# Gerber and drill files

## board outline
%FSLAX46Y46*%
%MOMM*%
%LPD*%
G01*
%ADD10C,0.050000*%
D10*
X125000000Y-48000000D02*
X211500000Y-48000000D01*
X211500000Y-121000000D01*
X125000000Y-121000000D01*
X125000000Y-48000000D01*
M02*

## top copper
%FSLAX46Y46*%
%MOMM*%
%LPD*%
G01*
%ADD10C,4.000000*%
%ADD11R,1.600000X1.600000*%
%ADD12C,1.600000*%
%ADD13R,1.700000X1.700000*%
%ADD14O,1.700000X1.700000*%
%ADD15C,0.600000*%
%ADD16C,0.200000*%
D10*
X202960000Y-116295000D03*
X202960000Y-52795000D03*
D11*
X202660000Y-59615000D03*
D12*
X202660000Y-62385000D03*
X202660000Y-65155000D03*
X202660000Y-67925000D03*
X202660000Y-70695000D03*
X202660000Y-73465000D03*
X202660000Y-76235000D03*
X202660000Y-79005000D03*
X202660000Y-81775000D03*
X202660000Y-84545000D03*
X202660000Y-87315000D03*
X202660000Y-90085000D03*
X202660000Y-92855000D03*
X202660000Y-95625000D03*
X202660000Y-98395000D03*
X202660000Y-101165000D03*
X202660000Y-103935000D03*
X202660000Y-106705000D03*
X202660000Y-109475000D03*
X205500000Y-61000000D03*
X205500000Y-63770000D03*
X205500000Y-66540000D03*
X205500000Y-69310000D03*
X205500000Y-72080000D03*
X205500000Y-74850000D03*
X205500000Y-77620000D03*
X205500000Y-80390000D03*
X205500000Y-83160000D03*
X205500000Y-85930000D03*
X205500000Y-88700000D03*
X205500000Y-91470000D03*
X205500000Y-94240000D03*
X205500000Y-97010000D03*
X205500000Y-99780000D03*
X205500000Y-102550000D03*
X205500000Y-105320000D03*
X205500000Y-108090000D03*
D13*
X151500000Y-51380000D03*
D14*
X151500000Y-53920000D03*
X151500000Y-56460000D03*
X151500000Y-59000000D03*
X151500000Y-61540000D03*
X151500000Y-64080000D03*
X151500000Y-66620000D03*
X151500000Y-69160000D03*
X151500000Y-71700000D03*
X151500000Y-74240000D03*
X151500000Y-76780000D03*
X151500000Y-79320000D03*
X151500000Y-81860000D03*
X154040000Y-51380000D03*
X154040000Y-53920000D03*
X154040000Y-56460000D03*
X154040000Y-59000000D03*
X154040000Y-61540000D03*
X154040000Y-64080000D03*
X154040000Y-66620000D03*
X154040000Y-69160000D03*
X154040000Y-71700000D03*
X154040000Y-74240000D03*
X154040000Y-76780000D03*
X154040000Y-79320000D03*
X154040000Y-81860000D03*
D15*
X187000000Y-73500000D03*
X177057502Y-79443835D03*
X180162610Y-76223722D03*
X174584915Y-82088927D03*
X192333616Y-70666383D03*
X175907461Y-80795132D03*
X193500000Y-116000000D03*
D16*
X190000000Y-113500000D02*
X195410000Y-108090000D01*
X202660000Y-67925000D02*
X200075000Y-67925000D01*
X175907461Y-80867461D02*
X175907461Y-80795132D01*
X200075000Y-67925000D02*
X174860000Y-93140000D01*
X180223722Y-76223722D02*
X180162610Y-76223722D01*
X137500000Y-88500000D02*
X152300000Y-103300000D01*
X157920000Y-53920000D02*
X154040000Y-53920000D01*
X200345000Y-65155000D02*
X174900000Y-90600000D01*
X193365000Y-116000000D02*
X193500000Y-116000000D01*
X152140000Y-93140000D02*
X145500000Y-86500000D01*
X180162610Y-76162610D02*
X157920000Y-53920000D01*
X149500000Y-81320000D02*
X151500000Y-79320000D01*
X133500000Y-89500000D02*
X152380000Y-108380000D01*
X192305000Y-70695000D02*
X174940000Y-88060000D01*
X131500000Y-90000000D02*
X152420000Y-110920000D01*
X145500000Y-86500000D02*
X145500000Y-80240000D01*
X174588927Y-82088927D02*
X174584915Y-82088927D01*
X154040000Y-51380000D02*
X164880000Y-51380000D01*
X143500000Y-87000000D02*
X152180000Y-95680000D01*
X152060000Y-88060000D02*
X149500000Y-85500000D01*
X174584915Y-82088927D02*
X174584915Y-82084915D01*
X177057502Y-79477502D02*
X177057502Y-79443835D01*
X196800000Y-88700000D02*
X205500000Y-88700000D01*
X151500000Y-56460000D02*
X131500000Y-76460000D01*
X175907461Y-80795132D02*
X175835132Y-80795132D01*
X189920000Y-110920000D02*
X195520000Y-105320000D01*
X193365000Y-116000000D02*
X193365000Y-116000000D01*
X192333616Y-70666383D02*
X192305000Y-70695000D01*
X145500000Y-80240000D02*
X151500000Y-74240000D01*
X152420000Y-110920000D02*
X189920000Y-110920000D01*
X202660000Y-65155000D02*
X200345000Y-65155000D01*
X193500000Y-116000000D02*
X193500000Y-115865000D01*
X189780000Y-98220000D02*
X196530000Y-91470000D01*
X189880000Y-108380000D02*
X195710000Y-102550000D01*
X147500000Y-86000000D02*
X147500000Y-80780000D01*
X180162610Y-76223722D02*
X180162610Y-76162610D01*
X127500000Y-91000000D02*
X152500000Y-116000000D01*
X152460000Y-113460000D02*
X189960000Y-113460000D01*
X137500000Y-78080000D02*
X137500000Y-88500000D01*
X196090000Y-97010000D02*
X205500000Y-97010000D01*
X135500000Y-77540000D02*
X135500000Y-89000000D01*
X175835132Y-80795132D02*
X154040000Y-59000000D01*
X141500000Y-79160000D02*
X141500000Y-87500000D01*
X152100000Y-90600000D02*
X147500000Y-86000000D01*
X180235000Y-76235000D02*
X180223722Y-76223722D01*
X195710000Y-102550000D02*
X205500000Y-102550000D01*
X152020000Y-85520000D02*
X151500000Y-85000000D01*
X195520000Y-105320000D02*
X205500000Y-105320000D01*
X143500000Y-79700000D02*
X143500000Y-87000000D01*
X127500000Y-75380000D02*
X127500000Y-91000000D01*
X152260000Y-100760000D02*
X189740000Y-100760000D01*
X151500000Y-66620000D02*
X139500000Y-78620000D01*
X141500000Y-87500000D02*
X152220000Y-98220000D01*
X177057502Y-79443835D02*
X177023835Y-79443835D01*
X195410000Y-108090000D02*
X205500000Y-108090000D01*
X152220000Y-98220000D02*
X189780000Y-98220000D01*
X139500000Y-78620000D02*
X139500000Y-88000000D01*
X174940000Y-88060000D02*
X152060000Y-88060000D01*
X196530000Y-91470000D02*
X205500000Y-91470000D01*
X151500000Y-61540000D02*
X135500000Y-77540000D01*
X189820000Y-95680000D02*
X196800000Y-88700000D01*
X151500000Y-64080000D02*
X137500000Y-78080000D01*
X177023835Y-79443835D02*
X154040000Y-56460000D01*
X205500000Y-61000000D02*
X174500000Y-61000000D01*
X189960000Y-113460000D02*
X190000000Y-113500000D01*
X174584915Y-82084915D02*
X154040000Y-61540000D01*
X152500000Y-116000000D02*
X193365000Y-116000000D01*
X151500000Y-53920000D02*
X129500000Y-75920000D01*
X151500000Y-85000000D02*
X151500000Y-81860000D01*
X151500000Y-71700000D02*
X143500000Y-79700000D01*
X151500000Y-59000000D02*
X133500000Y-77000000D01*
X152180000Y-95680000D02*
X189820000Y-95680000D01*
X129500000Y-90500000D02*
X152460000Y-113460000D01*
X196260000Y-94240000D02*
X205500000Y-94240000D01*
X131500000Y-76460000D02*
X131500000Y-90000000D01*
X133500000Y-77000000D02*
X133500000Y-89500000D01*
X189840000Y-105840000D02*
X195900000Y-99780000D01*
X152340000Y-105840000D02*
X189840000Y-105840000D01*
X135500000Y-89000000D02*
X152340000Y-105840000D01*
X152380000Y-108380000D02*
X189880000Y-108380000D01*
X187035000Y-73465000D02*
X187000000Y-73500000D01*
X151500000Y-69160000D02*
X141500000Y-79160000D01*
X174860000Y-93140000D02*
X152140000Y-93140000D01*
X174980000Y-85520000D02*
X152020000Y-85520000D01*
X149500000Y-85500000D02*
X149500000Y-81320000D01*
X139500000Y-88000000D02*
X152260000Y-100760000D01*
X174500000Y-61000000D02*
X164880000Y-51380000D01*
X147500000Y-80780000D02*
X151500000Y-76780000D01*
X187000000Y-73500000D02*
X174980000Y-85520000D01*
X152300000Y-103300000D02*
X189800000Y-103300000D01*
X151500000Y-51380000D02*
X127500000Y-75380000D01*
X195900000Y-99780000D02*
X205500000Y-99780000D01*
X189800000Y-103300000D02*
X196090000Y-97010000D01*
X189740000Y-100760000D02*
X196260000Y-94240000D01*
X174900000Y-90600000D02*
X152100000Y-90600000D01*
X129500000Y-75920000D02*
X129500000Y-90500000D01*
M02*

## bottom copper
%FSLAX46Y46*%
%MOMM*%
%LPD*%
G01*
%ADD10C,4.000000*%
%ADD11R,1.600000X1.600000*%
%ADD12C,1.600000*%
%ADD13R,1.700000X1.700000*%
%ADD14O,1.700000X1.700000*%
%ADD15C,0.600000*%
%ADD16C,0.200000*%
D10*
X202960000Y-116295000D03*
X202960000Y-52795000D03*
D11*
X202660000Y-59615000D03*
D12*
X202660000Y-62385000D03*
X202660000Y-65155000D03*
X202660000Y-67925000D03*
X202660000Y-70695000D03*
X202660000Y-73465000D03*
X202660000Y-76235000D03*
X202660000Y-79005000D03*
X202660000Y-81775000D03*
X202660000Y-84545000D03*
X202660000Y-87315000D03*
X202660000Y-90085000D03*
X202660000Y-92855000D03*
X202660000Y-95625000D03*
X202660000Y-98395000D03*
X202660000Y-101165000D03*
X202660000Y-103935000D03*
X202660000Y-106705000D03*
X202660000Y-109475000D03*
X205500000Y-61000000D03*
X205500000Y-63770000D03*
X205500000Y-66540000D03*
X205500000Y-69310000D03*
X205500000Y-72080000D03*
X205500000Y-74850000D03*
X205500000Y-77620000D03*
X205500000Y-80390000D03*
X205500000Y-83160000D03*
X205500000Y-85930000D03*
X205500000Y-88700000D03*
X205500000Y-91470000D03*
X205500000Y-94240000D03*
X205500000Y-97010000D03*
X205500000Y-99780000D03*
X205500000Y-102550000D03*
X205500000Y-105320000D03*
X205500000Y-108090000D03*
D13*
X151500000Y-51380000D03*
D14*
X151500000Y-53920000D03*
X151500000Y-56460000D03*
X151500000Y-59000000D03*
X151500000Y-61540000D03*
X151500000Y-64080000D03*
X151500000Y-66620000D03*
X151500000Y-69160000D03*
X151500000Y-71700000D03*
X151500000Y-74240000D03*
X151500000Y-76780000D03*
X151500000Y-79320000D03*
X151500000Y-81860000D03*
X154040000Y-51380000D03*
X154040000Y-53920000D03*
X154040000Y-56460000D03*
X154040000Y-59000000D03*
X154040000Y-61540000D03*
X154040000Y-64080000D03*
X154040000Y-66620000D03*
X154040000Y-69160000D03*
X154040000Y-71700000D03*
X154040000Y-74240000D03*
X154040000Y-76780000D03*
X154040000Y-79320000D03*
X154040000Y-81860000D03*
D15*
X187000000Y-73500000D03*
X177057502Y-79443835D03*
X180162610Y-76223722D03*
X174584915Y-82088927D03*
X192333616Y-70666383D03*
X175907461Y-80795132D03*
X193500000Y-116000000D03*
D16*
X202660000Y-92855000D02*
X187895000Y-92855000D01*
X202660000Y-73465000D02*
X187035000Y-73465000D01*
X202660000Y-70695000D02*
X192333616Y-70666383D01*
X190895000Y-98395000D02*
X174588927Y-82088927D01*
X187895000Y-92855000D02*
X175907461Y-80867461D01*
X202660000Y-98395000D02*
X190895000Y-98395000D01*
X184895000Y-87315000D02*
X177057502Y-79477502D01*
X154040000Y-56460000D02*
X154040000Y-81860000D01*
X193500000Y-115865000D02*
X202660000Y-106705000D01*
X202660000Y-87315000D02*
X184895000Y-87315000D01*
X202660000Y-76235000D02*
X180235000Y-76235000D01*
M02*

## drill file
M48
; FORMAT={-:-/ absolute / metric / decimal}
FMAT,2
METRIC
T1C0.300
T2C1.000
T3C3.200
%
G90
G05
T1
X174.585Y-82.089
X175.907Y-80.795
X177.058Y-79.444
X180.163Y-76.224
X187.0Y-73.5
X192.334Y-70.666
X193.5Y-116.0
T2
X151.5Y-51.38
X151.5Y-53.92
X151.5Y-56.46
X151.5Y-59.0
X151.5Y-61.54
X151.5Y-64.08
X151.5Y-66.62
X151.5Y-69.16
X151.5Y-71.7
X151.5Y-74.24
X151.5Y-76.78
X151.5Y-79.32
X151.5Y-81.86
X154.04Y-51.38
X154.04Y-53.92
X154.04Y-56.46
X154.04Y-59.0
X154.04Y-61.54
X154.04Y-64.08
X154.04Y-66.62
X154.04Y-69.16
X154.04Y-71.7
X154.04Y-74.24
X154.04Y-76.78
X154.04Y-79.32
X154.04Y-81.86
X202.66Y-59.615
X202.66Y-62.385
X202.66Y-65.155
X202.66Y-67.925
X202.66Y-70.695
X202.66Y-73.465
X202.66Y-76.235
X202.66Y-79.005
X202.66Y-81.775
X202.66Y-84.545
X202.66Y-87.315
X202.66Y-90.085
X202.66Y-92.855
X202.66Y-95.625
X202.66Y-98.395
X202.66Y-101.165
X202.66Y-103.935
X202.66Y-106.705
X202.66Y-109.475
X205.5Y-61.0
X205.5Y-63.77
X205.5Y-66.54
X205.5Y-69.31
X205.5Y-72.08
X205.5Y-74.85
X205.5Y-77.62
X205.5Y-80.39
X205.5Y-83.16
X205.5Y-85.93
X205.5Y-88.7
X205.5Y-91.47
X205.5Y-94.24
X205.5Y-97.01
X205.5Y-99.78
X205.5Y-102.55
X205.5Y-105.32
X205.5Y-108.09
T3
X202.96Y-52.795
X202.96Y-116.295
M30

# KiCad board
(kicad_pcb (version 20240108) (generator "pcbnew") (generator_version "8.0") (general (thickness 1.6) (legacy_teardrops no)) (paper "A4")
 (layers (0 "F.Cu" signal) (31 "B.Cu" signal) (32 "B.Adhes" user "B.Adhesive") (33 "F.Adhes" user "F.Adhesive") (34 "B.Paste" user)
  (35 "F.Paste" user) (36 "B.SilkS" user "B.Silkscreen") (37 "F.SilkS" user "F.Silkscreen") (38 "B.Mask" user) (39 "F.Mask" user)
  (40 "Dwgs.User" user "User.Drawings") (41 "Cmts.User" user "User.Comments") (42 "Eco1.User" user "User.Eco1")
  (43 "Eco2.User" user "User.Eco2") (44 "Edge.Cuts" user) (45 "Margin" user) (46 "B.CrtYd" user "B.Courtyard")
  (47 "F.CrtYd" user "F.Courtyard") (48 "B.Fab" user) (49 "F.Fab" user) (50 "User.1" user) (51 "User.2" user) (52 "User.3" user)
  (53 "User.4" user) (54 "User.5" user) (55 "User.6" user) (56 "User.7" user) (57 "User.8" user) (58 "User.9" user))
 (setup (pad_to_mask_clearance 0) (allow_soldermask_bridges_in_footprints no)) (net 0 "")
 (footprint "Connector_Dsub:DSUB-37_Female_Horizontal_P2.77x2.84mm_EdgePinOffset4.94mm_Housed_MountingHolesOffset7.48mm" (layer "F.Cu")
  (at 202.66 59.615 90)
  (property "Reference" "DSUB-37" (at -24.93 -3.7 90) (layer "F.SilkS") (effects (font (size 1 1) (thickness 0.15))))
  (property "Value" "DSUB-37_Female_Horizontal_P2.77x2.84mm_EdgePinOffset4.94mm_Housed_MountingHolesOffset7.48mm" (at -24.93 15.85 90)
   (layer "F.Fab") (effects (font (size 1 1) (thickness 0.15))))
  (pad "0" thru_hole circle (at -56.68 0.3 90) (size 4 4) (drill 3.2) (layers "*.Cu" "*.Mask") (remove_unused_layers no))
  (pad "0" thru_hole circle (at 6.82 0.3 90) (size 4 4) (drill 3.2) (layers "*.Cu" "*.Mask") (remove_unused_layers no))
  (pad "1" thru_hole rect (at 0 0 90) (size 1.6 1.6) (drill 1) (layers "*.Cu" "*.Mask") (remove_unused_layers no))
  (pad "2" thru_hole circle (at -2.77 0 90) (size 1.6 1.6) (drill 1) (layers "*.Cu" "*.Mask") (remove_unused_layers no))
  (pad "3" thru_hole circle (at -5.54 0 90) (size 1.6 1.6) (drill 1) (layers "*.Cu" "*.Mask") (remove_unused_layers no))
  (pad "4" thru_hole circle (at -8.31 0 90) (size 1.6 1.6) (drill 1) (layers "*.Cu" "*.Mask") (remove_unused_layers no))
  (pad "5" thru_hole circle (at -11.08 0 90) (size 1.6 1.6) (drill 1) (layers "*.Cu" "*.Mask") (remove_unused_layers no))
  (pad "6" thru_hole circle (at -13.85 0 90) (size 1.6 1.6) (drill 1) (layers "*.Cu" "*.Mask") (remove_unused_layers no))
  (pad "7" thru_hole circle (at -16.62 0 90) (size 1.6 1.6) (drill 1) (layers "*.Cu" "*.Mask") (remove_unused_layers no))
  (pad "8" thru_hole circle (at -19.39 0 90) (size 1.6 1.6) (drill 1) (layers "*.Cu" "*.Mask") (remove_unused_layers no))
  (pad "9" thru_hole circle (at -22.16 0 90) (size 1.6 1.6) (drill 1) (layers "*.Cu" "*.Mask") (remove_unused_layers no))
  (pad "10" thru_hole circle (at -24.93 0 90) (size 1.6 1.6) (drill 1) (layers "*.Cu" "*.Mask") (remove_unused_layers no))
  (pad "11" thru_hole circle (at -27.7 0 90) (size 1.6 1.6) (drill 1) (layers "*.Cu" "*.Mask") (remove_unused_layers no))
  (pad "12" thru_hole circle (at -30.47 0 90) (size 1.6 1.6) (drill 1) (layers "*.Cu" "*.Mask") (remove_unused_layers no))
  (pad "13" thru_hole circle (at -33.24 0 90) (size 1.6 1.6) (drill 1) (layers "*.Cu" "*.Mask") (remove_unused_layers no))
  (pad "14" thru_hole circle (at -36.01 0 90) (size 1.6 1.6) (drill 1) (layers "*.Cu" "*.Mask") (remove_unused_layers no))
  (pad "15" thru_hole circle (at -38.78 0 90) (size 1.6 1.6) (drill 1) (layers "*.Cu" "*.Mask") (remove_unused_layers no))
  (pad "16" thru_hole circle (at -41.55 0 90) (size 1.6 1.6) (drill 1) (layers "*.Cu" "*.Mask") (remove_unused_layers no))
  (pad "17" thru_hole circle (at -44.32 0 90) (size 1.6 1.6) (drill 1) (layers "*.Cu" "*.Mask") (remove_unused_layers no))
  (pad "18" thru_hole circle (at -47.09 0 90) (size 1.6 1.6) (drill 1) (layers "*.Cu" "*.Mask") (remove_unused_layers no))
  (pad "19" thru_hole circle (at -49.86 0 90) (size 1.6 1.6) (drill 1) (layers "*.Cu" "*.Mask") (remove_unused_layers no))
  (pad "20" thru_hole circle (at -1.385 2.84 90) (size 1.6 1.6) (drill 1) (layers "*.Cu" "*.Mask") (remove_unused_layers no))
  (pad "21" thru_hole circle (at -4.155 2.84 90) (size 1.6 1.6) (drill 1) (layers "*.Cu" "*.Mask") (remove_unused_layers no))
  (pad "22" thru_hole circle (at -6.925 2.84 90) (size 1.6 1.6) (drill 1) (layers "*.Cu" "*.Mask") (remove_unused_layers no))
  (pad "23" thru_hole circle (at -9.695 2.84 90) (size 1.6 1.6) (drill 1) (layers "*.Cu" "*.Mask") (remove_unused_layers no))
  (pad "24" thru_hole circle (at -12.465 2.84 90) (size 1.6 1.6) (drill 1) (layers "*.Cu" "*.Mask") (remove_unused_layers no))
  (pad "25" thru_hole circle (at -15.235 2.84 90) (size 1.6 1.6) (drill 1) (layers "*.Cu" "*.Mask") (remove_unused_layers no))
  (pad "26" thru_hole circle (at -18.005 2.84 90) (size 1.6 1.6) (drill 1) (layers "*.Cu" "*.Mask") (remove_unused_layers no))
  (pad "27" thru_hole circle (at -20.775 2.84 90) (size 1.6 1.6) (drill 1) (layers "*.Cu" "*.Mask") (remove_unused_layers no))
  (pad "28" thru_hole circle (at -23.545 2.84 90) (size 1.6 1.6) (drill 1) (layers "*.Cu" "*.Mask") (remove_unused_layers no))
  (pad "29" thru_hole circle (at -26.315 2.84 90) (size 1.6 1.6) (drill 1) (layers "*.Cu" "*.Mask") (remove_unused_layers no))
  (pad "30" thru_hole circle (at -29.085 2.84 90) (size 1.6 1.6) (drill 1) (layers "*.Cu" "*.Mask") (remove_unused_layers no))
  (pad "31" thru_hole circle (at -31.855 2.84 90) (size 1.6 1.6) (drill 1) (layers "*.Cu" "*.Mask") (remove_unused_layers no))
  (pad "32" thru_hole circle (at -34.625 2.84 90) (size 1.6 1.6) (drill 1) (layers "*.Cu" "*.Mask") (remove_unused_layers no))
  (pad "33" thru_hole circle (at -37.395 2.84 90) (size 1.6 1.6) (drill 1) (layers "*.Cu" "*.Mask") (remove_unused_layers no))
  (pad "34" thru_hole circle (at -40.165 2.84 90) (size 1.6 1.6) (drill 1) (layers "*.Cu" "*.Mask") (remove_unused_layers no))
  (pad "35" thru_hole circle (at -42.935 2.84 90) (size 1.6 1.6) (drill 1) (layers "*.Cu" "*.Mask") (remove_unused_layers no))
  (pad "36" thru_hole circle (at -45.705 2.84 90) (size 1.6 1.6) (drill 1) (layers "*.Cu" "*.Mask") (remove_unused_layers no))
  (pad "37" thru_hole circle (at -48.475 2.84 90) (size 1.6 1.6) (drill 1) (layers "*.Cu" "*.Mask") (remove_unused_layers no)))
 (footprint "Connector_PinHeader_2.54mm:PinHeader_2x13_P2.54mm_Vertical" (layer "F.Cu") (at 151.5 51.38)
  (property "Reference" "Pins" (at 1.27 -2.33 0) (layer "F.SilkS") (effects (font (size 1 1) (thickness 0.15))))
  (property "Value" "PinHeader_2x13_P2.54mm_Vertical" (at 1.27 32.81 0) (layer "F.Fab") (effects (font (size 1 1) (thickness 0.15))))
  (pad "1" thru_hole rect (at 0 0) (size 1.7 1.7) (drill 1) (layers "*.Cu" "*.Mask") (remove_unused_layers no))
  (pad "2" thru_hole oval (at 0 2.54) (size 1.7 1.7) (drill 1) (layers "*.Cu" "*.Mask") (remove_unused_layers no))
  (pad "3" thru_hole oval (at 0 5.08) (size 1.7 1.7) (drill 1) (layers "*.Cu" "*.Mask") (remove_unused_layers no))
  (pad "4" thru_hole oval (at 0 7.62) (size 1.7 1.7) (drill 1) (layers "*.Cu" "*.Mask") (remove_unused_layers no))
  (pad "5" thru_hole oval (at 0 10.16) (size 1.7 1.7) (drill 1) (layers "*.Cu" "*.Mask") (remove_unused_layers no))
  (pad "6" thru_hole oval (at 0 12.7) (size 1.7 1.7) (drill 1) (layers "*.Cu" "*.Mask") (remove_unused_layers no))
  (pad "7" thru_hole oval (at 0 15.24) (size 1.7 1.7) (drill 1) (layers "*.Cu" "*.Mask") (remove_unused_layers no))
  (pad "8" thru_hole oval (at 0 17.78) (size 1.7 1.7) (drill 1) (layers "*.Cu" "*.Mask") (remove_unused_layers no))
  (pad "9" thru_hole oval (at 0 20.32) (size 1.7 1.7) (drill 1) (layers "*.Cu" "*.Mask") (remove_unused_layers no))
  (pad "10" thru_hole oval (at 0 22.86) (size 1.7 1.7) (drill 1) (layers "*.Cu" "*.Mask") (remove_unused_layers no))
  (pad "11" thru_hole oval (at 0 25.4) (size 1.7 1.7) (drill 1) (layers "*.Cu" "*.Mask") (remove_unused_layers no))
  (pad "12" thru_hole oval (at 0 27.94) (size 1.7 1.7) (drill 1) (layers "*.Cu" "*.Mask") (remove_unused_layers no))
  (pad "13" thru_hole oval (at 0 30.48) (size 1.7 1.7) (drill 1) (layers "*.Cu" "*.Mask") (remove_unused_layers no))
  (pad "14" thru_hole oval (at 2.54 0) (size 1.7 1.7) (drill 1) (layers "*.Cu" "*.Mask") (remove_unused_layers no))
  (pad "15" thru_hole oval (at 2.54 2.54) (size 1.7 1.7) (drill 1) (layers "*.Cu" "*.Mask") (remove_unused_layers no))
  (pad "16" thru_hole oval (at 2.54 5.08) (size 1.7 1.7) (drill 1) (layers "*.Cu" "*.Mask") (remove_unused_layers no))
  (pad "17" thru_hole oval (at 2.54 7.62) (size 1.7 1.7) (drill 1) (layers "*.Cu" "*.Mask") (remove_unused_layers no))
  (pad "18" thru_hole oval (at 2.54 10.16) (size 1.7 1.7) (drill 1) (layers "*.Cu" "*.Mask") (remove_unused_layers no))
  (pad "19" thru_hole oval (at 2.54 12.7) (size 1.7 1.7) (drill 1) (layers "*.Cu" "*.Mask") (remove_unused_layers no))
  (pad "20" thru_hole oval (at 2.54 15.24) (size 1.7 1.7) (drill 1) (layers "*.Cu" "*.Mask") (remove_unused_layers no))
  (pad "21" thru_hole oval (at 2.54 17.78) (size 1.7 1.7) (drill 1) (layers "*.Cu" "*.Mask") (remove_unused_layers no))
  (pad "22" thru_hole oval (at 2.54 20.32) (size 1.7 1.7) (drill 1) (layers "*.Cu" "*.Mask") (remove_unused_layers no))
  (pad "23" thru_hole oval (at 2.54 22.86) (size 1.7 1.7) (drill 1) (layers "*.Cu" "*.Mask") (remove_unused_layers no))
  (pad "24" thru_hole oval (at 2.54 25.4) (size 1.7 1.7) (drill 1) (layers "*.Cu" "*.Mask") (remove_unused_layers no))
  (pad "25" thru_hole oval (at 2.54 27.94) (size 1.7 1.7) (drill 1) (layers "*.Cu" "*.Mask") (remove_unused_layers no))
  (pad "26" thru_hole oval (at 2.54 30.48) (size 1.7 1.7) (drill 1) (layers "*.Cu" "*.Mask") (remove_unused_layers no)))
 (gr_rect (start 125 48) (end 211.5 121) (stroke (width 0.05) (type default)) (fill none) (layer "Edge.Cuts"))
 (segment (start 190 113.5) (end 195.41 108.09) (width 0.2) (layer "F.Cu") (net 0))
 (segment (start 202.66 67.925) (end 200.075 67.925) (width 0.2) (layer "F.Cu") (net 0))
 (segment (start 175.907461 80.867461) (end 175.907461 80.795132) (width 0.2) (layer "F.Cu") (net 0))
 (segment (start 200.075 67.925) (end 174.86 93.14) (width 0.2) (layer "F.Cu") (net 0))
 (segment (start 180.223722 76.223722) (end 180.16261 76.223722) (width 0.2) (layer "F.Cu") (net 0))
 (segment (start 137.5 88.5) (end 152.3 103.3) (width 0.2) (layer "F.Cu") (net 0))
 (segment (start 157.92 53.92) (end 154.04 53.92) (width 0.2) (layer "F.Cu") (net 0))
 (segment (start 200.345 65.155) (end 174.9 90.6) (width 0.2) (layer "F.Cu") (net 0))
 (segment (start 193.365 116) (end 193.5 116) (width 0.2) (layer "F.Cu") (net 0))
 (segment (start 152.14 93.14) (end 145.5 86.5) (width 0.2) (layer "F.Cu") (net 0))
 (segment (start 180.16261 76.16261) (end 157.92 53.92) (width 0.2) (layer "F.Cu") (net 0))
 (segment (start 149.5 81.32) (end 151.5 79.32) (width 0.2) (layer "F.Cu") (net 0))
 (segment (start 133.5 89.5) (end 152.38 108.38) (width 0.2) (layer "F.Cu") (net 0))
 (segment (start 192.305 70.695) (end 174.94 88.06) (width 0.2) (layer "F.Cu") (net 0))
 (segment (start 131.5 90) (end 152.42 110.92) (width 0.2) (layer "F.Cu") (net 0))
 (segment (start 145.5 86.5) (end 145.5 80.24) (width 0.2) (layer "F.Cu") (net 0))
 (segment (start 174.588927 82.088927) (end 174.584915 82.088927) (width 0.2) (layer "F.Cu") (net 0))
 (segment (start 154.04 51.38) (end 164.88 51.38) (width 0.2) (layer "F.Cu") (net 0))
 (segment (start 143.5 87) (end 152.18 95.68) (width 0.2) (layer "F.Cu") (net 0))
 (segment (start 152.06 88.06) (end 149.5 85.5) (width 0.2) (layer "F.Cu") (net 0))
 (segment (start 174.584915 82.088927) (end 174.584915 82.084915) (width 0.2) (layer "F.Cu") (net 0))
 (segment (start 177.057502 79.477502) (end 177.057502 79.443835) (width 0.2) (layer "F.Cu") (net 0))
 (segment (start 196.8 88.7) (end 205.5 88.7) (width 0.2) (layer "F.Cu") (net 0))
 (segment (start 151.5 56.46) (end 131.5 76.46) (width 0.2) (layer "F.Cu") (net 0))
 (segment (start 175.907461 80.795132) (end 175.835132 80.795132) (width 0.2) (layer "F.Cu") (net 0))
 (segment (start 189.92 110.92) (end 195.52 105.32) (width 0.2) (layer "F.Cu") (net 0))
 (segment (start 193.365 116) (end 193.365 116) (width 0.2) (layer "F.Cu") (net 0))
 (segment (start 192.333616 70.666383) (end 192.305 70.695) (width 0.2) (layer "F.Cu") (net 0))
 (segment (start 145.5 80.24) (end 151.5 74.24) (width 0.2) (layer "F.Cu") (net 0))
 (segment (start 152.42 110.92) (end 189.92 110.92) (width 0.2) (layer "F.Cu") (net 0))
 (segment (start 202.66 65.155) (end 200.345 65.155) (width 0.2) (layer "F.Cu") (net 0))
 (segment (start 193.5 116) (end 193.5 115.865) (width 0.2) (layer "F.Cu") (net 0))
 (segment (start 189.78 98.22) (end 196.53 91.47) (width 0.2) (layer "F.Cu") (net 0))
 (segment (start 189.88 108.38) (end 195.71 102.55) (width 0.2) (layer "F.Cu") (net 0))
 (segment (start 147.5 86) (end 147.5 80.78) (width 0.2) (layer "F.Cu") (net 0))
 (segment (start 180.16261 76.223722) (end 180.16261 76.16261) (width 0.2) (layer "F.Cu") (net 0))
 (segment (start 127.5 91) (end 152.5 116) (width 0.2) (layer "F.Cu") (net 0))
 (segment (start 152.46 113.46) (end 189.96 113.46) (width 0.2) (layer "F.Cu") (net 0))
 (segment (start 137.5 78.08) (end 137.5 88.5) (width 0.2) (layer "F.Cu") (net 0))
 (segment (start 196.09 97.01) (end 205.5 97.01) (width 0.2) (layer "F.Cu") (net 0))
 (segment (start 135.5 77.54) (end 135.5 89) (width 0.2) (layer "F.Cu") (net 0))
 (segment (start 175.835132 80.795132) (end 154.04 59) (width 0.2) (layer "F.Cu") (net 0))
 (segment (start 141.5 79.16) (end 141.5 87.5) (width 0.2) (layer "F.Cu") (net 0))
 (segment (start 152.1 90.6) (end 147.5 86) (width 0.2) (layer "F.Cu") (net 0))
 (segment (start 180.235 76.235) (end 180.223722 76.223722) (width 0.2) (layer "F.Cu") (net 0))
 (segment (start 195.71 102.55) (end 205.5 102.55) (width 0.2) (layer "F.Cu") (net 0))
 (segment (start 152.02 85.52) (end 151.5 85) (width 0.2) (layer "F.Cu") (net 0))
 (segment (start 195.52 105.32) (end 205.5 105.32) (width 0.2) (layer "F.Cu") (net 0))
 (segment (start 143.5 79.7) (end 143.5 87) (width 0.2) (layer "F.Cu") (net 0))
 (segment (start 127.5 75.38) (end 127.5 91) (width 0.2) (layer "F.Cu") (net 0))
 (segment (start 152.26 100.76) (end 189.74 100.76) (width 0.2) (layer "F.Cu") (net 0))
 (segment (start 151.5 66.62) (end 139.5 78.62) (width 0.2) (layer "F.Cu") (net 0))
 (segment (start 141.5 87.5) (end 152.22 98.22) (width 0.2) (layer "F.Cu") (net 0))
 (segment (start 177.057502 79.443835) (end 177.023835 79.443835) (width 0.2) (layer "F.Cu") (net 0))
 (segment (start 195.41 108.09) (end 205.5 108.09) (width 0.2) (layer "F.Cu") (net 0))
 (segment (start 152.22 98.22) (end 189.78 98.22) (width 0.2) (layer "F.Cu") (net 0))
 (segment (start 139.5 78.62) (end 139.5 88) (width 0.2) (layer "F.Cu") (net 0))
 (segment (start 174.94 88.06) (end 152.06 88.06) (width 0.2) (layer "F.Cu") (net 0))
 (segment (start 196.53 91.47) (end 205.5 91.47) (width 0.2) (layer "F.Cu") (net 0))
 (segment (start 151.5 61.54) (end 135.5 77.54) (width 0.2) (layer "F.Cu") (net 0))
 (segment (start 189.82 95.68) (end 196.8 88.7) (width 0.2) (layer "F.Cu") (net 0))
 (segment (start 151.5 64.08) (end 137.5 78.08) (width 0.2) (layer "F.Cu") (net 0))
 (segment (start 177.023835 79.443835) (end 154.04 56.46) (width 0.2) (layer "F.Cu") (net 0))
 (segment (start 205.5 61) (end 174.5 61) (width 0.2) (layer "F.Cu") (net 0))
 (segment (start 189.96 113.46) (end 190 113.5) (width 0.2) (layer "F.Cu") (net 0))
 (segment (start 174.584915 82.084915) (end 154.04 61.54) (width 0.2) (layer "F.Cu") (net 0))
 (segment (start 152.5 116) (end 193.365 116) (width 0.2) (layer "F.Cu") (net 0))
 (segment (start 151.5 53.92) (end 129.5 75.92) (width 0.2) (layer "F.Cu") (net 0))
 (segment (start 151.5 85) (end 151.5 81.86) (width 0.2) (layer "F.Cu") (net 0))
 (segment (start 151.5 71.7) (end 143.5 79.7) (width 0.2) (layer "F.Cu") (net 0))
 (segment (start 151.5 59) (end 133.5 77) (width 0.2) (layer "F.Cu") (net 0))
 (segment (start 152.18 95.68) (end 189.82 95.68) (width 0.2) (layer "F.Cu") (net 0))
 (segment (start 129.5 90.5) (end 152.46 113.46) (width 0.2) (layer "F.Cu") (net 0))
 (segment (start 196.26 94.24) (end 205.5 94.24) (width 0.2) (layer "F.Cu") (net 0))
 (segment (start 131.5 76.46) (end 131.5 90) (width 0.2) (layer "F.Cu") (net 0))
 (segment (start 133.5 77) (end 133.5 89.5) (width 0.2) (layer "F.Cu") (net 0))
 (segment (start 189.84 105.84) (end 195.9 99.78) (width 0.2) (layer "F.Cu") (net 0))
 (segment (start 152.34 105.84) (end 189.84 105.84) (width 0.2) (layer "F.Cu") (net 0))
 (segment (start 135.5 89) (end 152.34 105.84) (width 0.2) (layer "F.Cu") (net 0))
 (segment (start 152.38 108.38) (end 189.88 108.38) (width 0.2) (layer "F.Cu") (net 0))
 (segment (start 187.035 73.465) (end 187 73.5) (width 0.2) (layer "F.Cu") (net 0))
 (segment (start 151.5 69.16) (end 141.5 79.16) (width 0.2) (layer "F.Cu") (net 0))
 (segment (start 174.86 93.14) (end 152.14 93.14) (width 0.2) (layer "F.Cu") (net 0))
 (segment (start 174.98 85.52) (end 152.02 85.52) (width 0.2) (layer "F.Cu") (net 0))
 (segment (start 149.5 85.5) (end 149.5 81.32) (width 0.2) (layer "F.Cu") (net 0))
 (segment (start 139.5 88) (end 152.26 100.76) (width 0.2) (layer "F.Cu") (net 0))
 (segment (start 174.5 61) (end 164.88 51.38) (width 0.2) (layer "F.Cu") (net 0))
 (segment (start 147.5 80.78) (end 151.5 76.78) (width 0.2) (layer "F.Cu") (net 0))
 (segment (start 187 73.5) (end 174.98 85.52) (width 0.2) (layer "F.Cu") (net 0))
 (segment (start 152.3 103.3) (end 189.8 103.3) (width 0.2) (layer "F.Cu") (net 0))
 (segment (start 151.5 51.38) (end 127.5 75.38) (width 0.2) (layer "F.Cu") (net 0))
 (segment (start 195.9 99.78) (end 205.5 99.78) (width 0.2) (layer "F.Cu") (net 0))
 (segment (start 189.8 103.3) (end 196.09 97.01) (width 0.2) (layer "F.Cu") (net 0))
 (segment (start 189.74 100.76) (end 196.26 94.24) (width 0.2) (layer "F.Cu") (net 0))
 (segment (start 174.9 90.6) (end 152.1 90.6) (width 0.2) (layer "F.Cu") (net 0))
 (segment (start 129.5 75.92) (end 129.5 90.5) (width 0.2) (layer "F.Cu") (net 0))
 (via (at 187 73.5) (size 0.6) (drill 0.3) (layers "F.Cu" "B.Cu") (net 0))
 (via (at 177.057502 79.443835) (size 0.6) (drill 0.3) (layers "F.Cu" "B.Cu") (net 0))
 (via (at 180.16261 76.223722) (size 0.6) (drill 0.3) (layers "F.Cu" "B.Cu") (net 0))
 (via (at 174.584915 82.088927) (size 0.6) (drill 0.3) (layers "F.Cu" "B.Cu") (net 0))
 (via (at 192.333616 70.666383) (size 0.6) (drill 0.3) (layers "F.Cu" "B.Cu") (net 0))
 (via (at 175.907461 80.795132) (size 0.6) (drill 0.3) (layers "F.Cu" "B.Cu") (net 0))
 (via (at 193.5 116) (size 0.6) (drill 0.3) (layers "F.Cu" "B.Cu") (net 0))
 (segment (start 202.66 92.855) (end 187.895 92.855) (width 0.2) (layer "B.Cu") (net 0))
 (segment (start 202.66 73.465) (end 187.035 73.465) (width 0.2) (layer "B.Cu") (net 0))
 (segment (start 202.66 70.695) (end 192.333616 70.666383) (width 0.2) (layer "B.Cu") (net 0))
 (segment (start 190.895 98.395) (end 174.588927 82.088927) (width 0.2) (layer "B.Cu") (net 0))
 (segment (start 187.895 92.855) (end 175.907461 80.867461) (width 0.2) (layer "B.Cu") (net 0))
 (segment (start 202.66 98.395) (end 190.895 98.395) (width 0.2) (layer "B.Cu") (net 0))
 (segment (start 184.895 87.315) (end 177.057502 79.477502) (width 0.2) (layer "B.Cu") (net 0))
 (segment (start 154.04 56.46) (end 154.04 81.86) (width 0.2) (layer "B.Cu") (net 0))
 (segment (start 193.5 115.865) (end 202.66 106.705) (width 0.2) (layer "B.Cu") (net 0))
 (segment (start 202.66 87.315) (end 184.895 87.315) (width 0.2) (layer "B.Cu") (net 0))
 (segment (start 202.66 76.235) (end 180.235 76.235) (width 0.2) (layer "B.Cu") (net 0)))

